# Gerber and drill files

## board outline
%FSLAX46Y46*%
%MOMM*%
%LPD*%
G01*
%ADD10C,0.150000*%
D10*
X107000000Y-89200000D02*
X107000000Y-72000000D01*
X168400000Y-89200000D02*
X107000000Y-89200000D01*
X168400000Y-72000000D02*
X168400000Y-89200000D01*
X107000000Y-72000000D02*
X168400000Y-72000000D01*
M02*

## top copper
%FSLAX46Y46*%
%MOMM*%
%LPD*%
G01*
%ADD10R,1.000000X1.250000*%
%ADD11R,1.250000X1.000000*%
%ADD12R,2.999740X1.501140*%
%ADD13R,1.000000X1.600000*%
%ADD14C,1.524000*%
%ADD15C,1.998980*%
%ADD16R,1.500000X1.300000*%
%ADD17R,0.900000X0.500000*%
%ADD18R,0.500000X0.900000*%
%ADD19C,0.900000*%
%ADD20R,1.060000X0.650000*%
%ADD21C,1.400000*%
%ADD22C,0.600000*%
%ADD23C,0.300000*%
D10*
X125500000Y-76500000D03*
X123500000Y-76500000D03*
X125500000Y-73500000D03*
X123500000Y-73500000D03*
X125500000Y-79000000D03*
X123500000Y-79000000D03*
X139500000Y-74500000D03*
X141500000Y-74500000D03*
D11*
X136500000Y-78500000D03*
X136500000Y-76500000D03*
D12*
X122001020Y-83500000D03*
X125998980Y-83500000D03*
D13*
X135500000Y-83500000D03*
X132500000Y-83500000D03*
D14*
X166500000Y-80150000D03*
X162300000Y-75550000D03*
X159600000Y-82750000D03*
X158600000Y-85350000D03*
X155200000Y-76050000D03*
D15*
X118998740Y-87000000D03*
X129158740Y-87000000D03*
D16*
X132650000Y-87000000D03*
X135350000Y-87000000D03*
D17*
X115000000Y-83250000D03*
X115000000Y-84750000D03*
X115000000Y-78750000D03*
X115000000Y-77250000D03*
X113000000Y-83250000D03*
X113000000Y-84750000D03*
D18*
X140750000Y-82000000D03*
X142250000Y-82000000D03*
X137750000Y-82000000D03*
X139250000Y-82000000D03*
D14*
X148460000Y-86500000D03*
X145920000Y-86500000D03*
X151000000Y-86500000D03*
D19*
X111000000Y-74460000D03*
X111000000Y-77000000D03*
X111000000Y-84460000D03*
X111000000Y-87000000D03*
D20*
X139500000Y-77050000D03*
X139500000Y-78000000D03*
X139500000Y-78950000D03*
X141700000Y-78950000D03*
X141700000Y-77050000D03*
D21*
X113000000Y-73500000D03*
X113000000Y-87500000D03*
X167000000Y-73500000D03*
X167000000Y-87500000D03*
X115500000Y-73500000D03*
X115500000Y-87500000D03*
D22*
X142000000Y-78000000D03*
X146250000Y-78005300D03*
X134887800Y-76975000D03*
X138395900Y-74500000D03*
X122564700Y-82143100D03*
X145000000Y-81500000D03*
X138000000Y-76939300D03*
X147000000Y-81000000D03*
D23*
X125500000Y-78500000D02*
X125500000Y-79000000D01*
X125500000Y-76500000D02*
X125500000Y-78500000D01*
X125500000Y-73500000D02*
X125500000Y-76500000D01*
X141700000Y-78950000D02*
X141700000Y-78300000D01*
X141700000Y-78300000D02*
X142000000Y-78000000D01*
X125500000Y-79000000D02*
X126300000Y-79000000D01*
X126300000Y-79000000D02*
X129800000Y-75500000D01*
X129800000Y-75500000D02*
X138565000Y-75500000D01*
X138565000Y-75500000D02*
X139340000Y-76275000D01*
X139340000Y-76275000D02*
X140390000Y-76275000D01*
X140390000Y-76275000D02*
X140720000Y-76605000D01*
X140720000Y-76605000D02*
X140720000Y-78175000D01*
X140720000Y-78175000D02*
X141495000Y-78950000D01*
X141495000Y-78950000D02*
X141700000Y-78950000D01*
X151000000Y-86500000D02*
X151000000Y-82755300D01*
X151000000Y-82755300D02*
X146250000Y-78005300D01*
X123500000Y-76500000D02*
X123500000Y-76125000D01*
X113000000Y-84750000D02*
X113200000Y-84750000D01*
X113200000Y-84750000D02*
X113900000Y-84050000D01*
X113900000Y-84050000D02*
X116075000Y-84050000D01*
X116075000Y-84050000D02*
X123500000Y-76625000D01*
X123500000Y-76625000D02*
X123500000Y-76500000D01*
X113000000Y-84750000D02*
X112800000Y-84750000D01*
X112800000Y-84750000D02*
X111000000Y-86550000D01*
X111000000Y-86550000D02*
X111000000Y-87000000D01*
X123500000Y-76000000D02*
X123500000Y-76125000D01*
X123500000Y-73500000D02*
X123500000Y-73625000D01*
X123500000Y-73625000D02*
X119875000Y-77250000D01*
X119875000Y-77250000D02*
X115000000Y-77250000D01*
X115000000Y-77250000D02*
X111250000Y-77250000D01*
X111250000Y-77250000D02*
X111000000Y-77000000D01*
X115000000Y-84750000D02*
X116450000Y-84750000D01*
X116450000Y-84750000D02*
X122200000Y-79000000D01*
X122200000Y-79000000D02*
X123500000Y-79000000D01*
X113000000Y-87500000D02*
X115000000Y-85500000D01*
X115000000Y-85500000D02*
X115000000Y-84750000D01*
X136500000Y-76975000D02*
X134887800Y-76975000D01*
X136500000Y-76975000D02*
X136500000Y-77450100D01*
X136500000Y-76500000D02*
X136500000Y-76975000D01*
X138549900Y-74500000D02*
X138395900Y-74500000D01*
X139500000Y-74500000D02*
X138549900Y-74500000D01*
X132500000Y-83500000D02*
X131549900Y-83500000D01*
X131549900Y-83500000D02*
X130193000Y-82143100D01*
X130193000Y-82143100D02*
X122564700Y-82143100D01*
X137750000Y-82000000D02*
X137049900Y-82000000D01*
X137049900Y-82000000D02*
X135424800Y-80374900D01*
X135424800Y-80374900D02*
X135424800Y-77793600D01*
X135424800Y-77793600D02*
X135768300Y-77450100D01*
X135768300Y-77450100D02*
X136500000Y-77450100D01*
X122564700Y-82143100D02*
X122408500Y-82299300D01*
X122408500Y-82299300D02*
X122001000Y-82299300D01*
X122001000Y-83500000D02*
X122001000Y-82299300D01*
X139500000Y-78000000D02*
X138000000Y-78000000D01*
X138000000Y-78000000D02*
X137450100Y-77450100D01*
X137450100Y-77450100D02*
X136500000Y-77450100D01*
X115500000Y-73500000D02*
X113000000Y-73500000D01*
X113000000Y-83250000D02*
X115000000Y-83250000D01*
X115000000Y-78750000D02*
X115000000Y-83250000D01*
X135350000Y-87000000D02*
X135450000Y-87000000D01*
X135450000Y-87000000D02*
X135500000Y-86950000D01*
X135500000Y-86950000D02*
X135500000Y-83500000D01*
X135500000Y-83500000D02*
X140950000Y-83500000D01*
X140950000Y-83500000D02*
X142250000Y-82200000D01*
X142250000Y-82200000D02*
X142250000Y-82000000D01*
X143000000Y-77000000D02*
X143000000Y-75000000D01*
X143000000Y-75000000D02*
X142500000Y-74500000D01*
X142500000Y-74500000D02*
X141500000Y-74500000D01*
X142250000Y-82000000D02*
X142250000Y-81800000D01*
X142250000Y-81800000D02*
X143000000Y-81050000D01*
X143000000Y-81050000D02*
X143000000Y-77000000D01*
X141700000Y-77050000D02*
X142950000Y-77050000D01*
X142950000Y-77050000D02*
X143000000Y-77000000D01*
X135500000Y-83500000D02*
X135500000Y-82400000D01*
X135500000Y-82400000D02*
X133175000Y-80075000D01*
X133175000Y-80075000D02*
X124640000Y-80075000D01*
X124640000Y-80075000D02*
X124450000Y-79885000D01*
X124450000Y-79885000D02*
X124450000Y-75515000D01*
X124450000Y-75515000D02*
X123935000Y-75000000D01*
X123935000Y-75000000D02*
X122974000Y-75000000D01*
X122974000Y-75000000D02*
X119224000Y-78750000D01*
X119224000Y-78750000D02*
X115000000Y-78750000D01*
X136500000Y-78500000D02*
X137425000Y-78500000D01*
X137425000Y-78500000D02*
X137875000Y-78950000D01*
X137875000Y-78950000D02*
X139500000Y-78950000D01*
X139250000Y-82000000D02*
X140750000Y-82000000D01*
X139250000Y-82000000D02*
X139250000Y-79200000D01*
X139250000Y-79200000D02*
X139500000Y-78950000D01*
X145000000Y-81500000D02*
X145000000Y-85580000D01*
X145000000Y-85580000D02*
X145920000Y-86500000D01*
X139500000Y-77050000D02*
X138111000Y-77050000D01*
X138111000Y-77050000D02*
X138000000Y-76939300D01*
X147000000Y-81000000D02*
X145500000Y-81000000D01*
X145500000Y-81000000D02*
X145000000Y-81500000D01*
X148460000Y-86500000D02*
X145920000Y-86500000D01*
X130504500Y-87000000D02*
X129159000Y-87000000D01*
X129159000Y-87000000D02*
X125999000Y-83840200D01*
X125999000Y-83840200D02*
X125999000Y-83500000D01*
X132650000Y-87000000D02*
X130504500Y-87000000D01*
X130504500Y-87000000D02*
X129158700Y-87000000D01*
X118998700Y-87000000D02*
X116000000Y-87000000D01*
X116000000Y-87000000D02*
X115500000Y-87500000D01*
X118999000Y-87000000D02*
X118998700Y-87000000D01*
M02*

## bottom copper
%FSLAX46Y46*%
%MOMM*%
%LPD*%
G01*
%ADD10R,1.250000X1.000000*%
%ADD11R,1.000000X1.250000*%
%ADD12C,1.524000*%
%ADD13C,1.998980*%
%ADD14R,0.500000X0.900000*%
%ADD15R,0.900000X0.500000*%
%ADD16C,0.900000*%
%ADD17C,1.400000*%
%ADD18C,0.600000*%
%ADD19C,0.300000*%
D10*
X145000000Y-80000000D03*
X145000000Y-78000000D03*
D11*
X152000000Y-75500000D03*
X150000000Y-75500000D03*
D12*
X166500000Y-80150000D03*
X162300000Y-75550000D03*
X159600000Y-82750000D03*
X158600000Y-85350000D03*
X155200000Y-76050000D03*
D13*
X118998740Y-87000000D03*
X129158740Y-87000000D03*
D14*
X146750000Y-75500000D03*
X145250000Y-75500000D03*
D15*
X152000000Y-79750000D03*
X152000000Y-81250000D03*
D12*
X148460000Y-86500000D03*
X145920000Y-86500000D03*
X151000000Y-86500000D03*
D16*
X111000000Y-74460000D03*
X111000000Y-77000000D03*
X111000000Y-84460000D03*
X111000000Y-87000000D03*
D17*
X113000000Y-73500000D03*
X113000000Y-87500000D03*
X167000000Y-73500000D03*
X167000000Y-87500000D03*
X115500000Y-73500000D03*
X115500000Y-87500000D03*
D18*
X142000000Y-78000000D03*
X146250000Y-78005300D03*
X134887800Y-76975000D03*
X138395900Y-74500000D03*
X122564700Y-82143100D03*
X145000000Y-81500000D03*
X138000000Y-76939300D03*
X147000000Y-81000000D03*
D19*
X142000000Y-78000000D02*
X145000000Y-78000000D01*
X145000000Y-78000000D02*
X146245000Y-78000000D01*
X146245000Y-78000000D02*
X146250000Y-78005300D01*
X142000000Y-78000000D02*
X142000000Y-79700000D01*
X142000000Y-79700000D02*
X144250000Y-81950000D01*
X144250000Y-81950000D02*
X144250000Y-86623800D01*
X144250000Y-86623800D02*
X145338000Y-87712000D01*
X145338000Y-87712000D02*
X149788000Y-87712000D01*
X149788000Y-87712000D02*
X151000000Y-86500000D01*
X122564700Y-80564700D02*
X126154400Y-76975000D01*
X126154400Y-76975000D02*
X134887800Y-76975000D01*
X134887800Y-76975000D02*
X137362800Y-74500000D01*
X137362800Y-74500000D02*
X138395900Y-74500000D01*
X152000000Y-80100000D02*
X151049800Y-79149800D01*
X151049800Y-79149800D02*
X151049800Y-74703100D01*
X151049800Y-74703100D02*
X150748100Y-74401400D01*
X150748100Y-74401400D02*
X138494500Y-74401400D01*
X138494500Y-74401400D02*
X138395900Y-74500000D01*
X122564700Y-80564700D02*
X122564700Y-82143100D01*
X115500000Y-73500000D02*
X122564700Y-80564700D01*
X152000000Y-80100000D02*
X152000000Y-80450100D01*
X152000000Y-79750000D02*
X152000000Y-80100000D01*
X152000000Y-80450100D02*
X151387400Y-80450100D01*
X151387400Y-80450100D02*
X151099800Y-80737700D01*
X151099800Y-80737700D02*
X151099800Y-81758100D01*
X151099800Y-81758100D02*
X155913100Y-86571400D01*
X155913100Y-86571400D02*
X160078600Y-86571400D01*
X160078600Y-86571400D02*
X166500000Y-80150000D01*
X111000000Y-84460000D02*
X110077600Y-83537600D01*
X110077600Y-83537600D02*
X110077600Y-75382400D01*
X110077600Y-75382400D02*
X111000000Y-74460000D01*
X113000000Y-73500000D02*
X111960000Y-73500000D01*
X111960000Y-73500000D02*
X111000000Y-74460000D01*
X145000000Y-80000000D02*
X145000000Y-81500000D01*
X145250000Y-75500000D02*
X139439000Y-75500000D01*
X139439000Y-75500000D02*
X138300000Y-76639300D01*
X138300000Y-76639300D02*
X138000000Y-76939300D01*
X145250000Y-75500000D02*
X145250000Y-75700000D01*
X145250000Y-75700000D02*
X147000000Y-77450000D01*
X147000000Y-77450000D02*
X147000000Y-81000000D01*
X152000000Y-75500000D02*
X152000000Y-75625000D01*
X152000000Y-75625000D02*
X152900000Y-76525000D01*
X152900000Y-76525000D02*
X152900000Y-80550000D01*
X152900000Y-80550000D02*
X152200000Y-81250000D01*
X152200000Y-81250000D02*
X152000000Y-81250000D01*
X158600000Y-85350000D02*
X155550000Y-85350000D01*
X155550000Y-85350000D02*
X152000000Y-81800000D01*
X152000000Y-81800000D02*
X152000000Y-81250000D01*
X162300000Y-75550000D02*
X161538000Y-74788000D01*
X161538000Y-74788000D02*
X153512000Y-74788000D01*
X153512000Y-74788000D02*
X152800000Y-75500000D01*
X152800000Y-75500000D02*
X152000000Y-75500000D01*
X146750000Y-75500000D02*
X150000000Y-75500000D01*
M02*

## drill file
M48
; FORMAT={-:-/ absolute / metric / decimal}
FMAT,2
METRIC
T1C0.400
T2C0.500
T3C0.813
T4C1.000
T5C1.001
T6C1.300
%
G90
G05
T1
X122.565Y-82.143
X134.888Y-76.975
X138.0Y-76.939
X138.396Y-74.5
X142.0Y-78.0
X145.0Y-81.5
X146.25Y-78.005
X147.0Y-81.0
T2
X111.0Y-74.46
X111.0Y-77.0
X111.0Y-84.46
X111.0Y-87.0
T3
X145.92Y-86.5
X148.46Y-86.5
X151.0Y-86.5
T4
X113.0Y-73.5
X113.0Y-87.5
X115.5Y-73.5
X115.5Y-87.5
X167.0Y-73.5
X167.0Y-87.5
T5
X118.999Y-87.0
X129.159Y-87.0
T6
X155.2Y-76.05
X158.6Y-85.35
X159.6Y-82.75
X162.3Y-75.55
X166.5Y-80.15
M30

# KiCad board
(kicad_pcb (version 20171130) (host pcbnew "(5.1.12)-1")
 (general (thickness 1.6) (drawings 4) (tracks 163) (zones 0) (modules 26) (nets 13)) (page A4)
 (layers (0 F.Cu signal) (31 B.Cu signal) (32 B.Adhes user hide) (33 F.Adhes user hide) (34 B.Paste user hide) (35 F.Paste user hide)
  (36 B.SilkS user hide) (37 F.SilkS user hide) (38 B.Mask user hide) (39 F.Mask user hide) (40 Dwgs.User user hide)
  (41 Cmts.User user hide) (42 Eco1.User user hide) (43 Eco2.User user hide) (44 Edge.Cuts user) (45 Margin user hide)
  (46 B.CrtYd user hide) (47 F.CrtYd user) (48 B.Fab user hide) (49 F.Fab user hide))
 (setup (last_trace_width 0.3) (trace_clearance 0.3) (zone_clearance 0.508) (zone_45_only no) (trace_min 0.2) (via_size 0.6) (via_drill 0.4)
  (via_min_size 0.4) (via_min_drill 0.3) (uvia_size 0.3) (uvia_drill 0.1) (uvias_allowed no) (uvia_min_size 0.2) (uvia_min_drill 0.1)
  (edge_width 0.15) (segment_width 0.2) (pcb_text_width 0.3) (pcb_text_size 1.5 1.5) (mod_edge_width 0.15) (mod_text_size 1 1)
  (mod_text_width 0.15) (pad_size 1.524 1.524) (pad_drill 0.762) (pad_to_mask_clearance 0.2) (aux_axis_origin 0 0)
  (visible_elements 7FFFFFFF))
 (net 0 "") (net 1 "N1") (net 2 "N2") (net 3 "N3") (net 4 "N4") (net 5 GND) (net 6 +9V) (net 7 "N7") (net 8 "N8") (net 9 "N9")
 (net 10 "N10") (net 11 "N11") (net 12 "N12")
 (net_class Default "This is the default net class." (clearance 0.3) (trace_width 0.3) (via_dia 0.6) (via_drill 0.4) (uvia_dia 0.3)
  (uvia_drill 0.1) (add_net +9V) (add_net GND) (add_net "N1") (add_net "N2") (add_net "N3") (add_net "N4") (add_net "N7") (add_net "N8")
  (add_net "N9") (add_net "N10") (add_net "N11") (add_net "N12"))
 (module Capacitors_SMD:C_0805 (layer F.Cu) (at 124.5 76.5 180)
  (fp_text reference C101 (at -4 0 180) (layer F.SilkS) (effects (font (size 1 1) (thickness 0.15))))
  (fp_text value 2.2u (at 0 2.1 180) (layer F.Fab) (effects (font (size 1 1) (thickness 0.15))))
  (pad 1 smd rect (at -1 0 180) (size 1 1.25) (layers F.Cu F.Paste F.Mask) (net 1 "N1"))
  (pad 2 smd rect (at 1 0 180) (size 1 1.25) (layers F.Cu F.Paste F.Mask) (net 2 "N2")))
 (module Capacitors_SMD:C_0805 (layer F.Cu) (at 124.5 73.5 180)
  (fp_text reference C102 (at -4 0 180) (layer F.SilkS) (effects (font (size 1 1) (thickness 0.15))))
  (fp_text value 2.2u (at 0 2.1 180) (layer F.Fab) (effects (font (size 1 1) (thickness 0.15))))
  (pad 1 smd rect (at -1 0 180) (size 1 1.25) (layers F.Cu F.Paste F.Mask) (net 1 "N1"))
  (pad 2 smd rect (at 1 0 180) (size 1 1.25) (layers F.Cu F.Paste F.Mask) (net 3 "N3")))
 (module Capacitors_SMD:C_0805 (layer F.Cu) (at 124.5 79 180)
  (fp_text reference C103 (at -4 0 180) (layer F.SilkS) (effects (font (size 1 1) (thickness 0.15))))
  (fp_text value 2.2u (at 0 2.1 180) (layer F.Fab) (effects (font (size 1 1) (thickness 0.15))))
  (pad 1 smd rect (at -1 0 180) (size 1 1.25) (layers F.Cu F.Paste F.Mask) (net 1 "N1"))
  (pad 2 smd rect (at 1 0 180) (size 1 1.25) (layers F.Cu F.Paste F.Mask) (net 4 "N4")))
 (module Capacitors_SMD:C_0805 (layer F.Cu) (at 140.5 74.5)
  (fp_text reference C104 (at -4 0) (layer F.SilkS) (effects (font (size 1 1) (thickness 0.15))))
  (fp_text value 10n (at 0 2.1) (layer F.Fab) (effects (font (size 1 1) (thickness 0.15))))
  (pad 1 smd rect (at -1 0) (size 1 1.25) (layers F.Cu F.Paste F.Mask) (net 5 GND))
  (pad 2 smd rect (at 1 0) (size 1 1.25) (layers F.Cu F.Paste F.Mask) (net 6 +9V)))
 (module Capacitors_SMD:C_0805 (layer F.Cu) (at 136.5 77.5 90)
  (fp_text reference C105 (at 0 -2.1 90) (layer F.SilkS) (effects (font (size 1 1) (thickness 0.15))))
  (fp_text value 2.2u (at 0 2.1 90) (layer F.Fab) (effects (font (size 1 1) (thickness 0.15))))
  (pad 1 smd rect (at -1 0 90) (size 1 1.25) (layers F.Cu F.Paste F.Mask) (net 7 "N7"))
  (pad 2 smd rect (at 1 0 90) (size 1 1.25) (layers F.Cu F.Paste F.Mask) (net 5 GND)))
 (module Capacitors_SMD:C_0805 (layer B.Cu) (at 145 79 90)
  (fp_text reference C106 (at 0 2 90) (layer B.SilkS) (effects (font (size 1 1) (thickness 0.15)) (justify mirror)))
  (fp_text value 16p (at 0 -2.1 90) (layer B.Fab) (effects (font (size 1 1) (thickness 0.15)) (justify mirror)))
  (pad 1 smd rect (at -1 0 90) (size 1 1.25) (layers B.Cu B.Paste B.Mask) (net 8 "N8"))
  (pad 2 smd rect (at 1 0 90) (size 1 1.25) (layers B.Cu B.Paste B.Mask) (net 1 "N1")))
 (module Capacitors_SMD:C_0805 (layer B.Cu) (at 151 75.5 180)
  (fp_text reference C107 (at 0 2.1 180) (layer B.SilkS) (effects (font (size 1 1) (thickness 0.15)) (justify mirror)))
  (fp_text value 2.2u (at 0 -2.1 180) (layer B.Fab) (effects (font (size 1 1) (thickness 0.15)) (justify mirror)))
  (pad 1 smd rect (at -1 0 180) (size 1 1.25) (layers B.Cu B.Paste B.Mask) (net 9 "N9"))
  (pad 2 smd rect (at 1 0 180) (size 1 1.25) (layers B.Cu B.Paste B.Mask) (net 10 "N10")))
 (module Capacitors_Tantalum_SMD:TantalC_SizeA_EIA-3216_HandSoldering (layer F.Cu) (at 124 83.5 180)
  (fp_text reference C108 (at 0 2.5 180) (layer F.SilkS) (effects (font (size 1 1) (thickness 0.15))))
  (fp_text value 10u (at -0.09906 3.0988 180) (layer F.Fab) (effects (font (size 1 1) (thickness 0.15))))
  (pad 2 smd rect (at 1.99898 0 180) (size 2.99974 1.50114) (layers F.Cu F.Paste F.Mask) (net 5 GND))
  (pad 1 smd rect (at -1.99898 0 180) (size 2.99974 1.50114) (layers F.Cu F.Paste F.Mask) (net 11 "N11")))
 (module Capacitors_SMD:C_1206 (layer F.Cu) (at 134 83.5 180)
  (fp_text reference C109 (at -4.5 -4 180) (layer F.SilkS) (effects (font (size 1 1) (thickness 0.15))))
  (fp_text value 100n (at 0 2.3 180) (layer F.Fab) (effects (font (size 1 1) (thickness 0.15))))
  (pad 1 smd rect (at -1.5 0 180) (size 1 1.6) (layers F.Cu F.Paste F.Mask) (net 6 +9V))
  (pad 2 smd rect (at 1.5 0 180) (size 1 1.6) (layers F.Cu F.Paste F.Mask) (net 5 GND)))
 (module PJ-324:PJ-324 (layer F.Cu) (at 168.2 86.15 180)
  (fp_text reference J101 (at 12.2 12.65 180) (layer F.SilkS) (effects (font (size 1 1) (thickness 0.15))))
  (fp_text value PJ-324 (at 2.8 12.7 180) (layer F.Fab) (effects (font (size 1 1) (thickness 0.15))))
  (pad 1 thru_hole circle (at 1.7 6 180) (size 1.524 1.524) (drill 1.3) (layers *.Cu *.Mask) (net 5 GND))
  (pad 5 thru_hole circle (at 5.9 10.6 180) (size 1.524 1.524) (drill 1.3) (layers *.Cu *.Mask) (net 9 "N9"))
  (pad 3 thru_hole circle (at 8.6 3.4 180) (size 1.524 1.524) (drill 1.3) (layers *.Cu *.Mask))
  (pad 2 thru_hole circle (at 9.6 0.8 180) (size 1.524 1.524) (drill 1.3) (layers *.Cu *.Mask) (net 9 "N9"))
  (pad 4 thru_hole circle (at 13 10.1 180) (size 1.524 1.524) (drill 1.3) (layers *.Cu *.Mask)))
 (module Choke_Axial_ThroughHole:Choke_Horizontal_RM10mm (layer F.Cu) (at 124 87)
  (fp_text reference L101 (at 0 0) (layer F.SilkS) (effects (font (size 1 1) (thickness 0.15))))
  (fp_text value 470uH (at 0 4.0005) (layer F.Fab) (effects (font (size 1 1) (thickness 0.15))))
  (pad 1 thru_hole circle (at -5.00126 0) (size 1.99898 1.99898) (drill 1.00076) (layers *.Cu *.Mask F.SilkS) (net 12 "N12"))
  (pad 2 thru_hole circle (at 5.15874 0) (size 1.99898 1.99898) (drill 1.00076) (layers *.Cu *.Mask F.SilkS) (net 11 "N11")))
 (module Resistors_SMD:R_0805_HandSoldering (layer F.Cu) (at 134 87)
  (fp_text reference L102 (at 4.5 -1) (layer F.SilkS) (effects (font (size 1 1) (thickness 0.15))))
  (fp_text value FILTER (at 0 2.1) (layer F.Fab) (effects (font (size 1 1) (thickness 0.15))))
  (pad 1 smd rect (at -1.35 0) (size 1.5 1.3) (layers F.Cu F.Paste F.Mask) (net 11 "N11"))
  (pad 2 smd rect (at 1.35 0) (size 1.5 1.3) (layers F.Cu F.Paste F.Mask) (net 6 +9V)))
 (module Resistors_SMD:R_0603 (layer F.Cu) (at 115 84 270)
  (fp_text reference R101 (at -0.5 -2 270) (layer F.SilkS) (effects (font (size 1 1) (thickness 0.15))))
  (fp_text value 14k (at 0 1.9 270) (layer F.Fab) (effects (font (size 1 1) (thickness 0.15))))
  (pad 1 smd rect (at -0.75 0 270) (size 0.5 0.9) (layers F.Cu F.Paste F.Mask) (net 6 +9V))
  (pad 2 smd rect (at 0.75 0 270) (size 0.5 0.9) (layers F.Cu F.Paste F.Mask) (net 4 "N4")))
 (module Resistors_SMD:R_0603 (layer F.Cu) (at 115 78 90)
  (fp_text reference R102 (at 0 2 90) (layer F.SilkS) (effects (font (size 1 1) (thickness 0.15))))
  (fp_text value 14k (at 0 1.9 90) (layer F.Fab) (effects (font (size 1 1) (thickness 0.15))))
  (pad 1 smd rect (at -0.75 0 90) (size 0.5 0.9) (layers F.Cu F.Paste F.Mask) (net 6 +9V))
  (pad 2 smd rect (at 0.75 0 90) (size 0.5 0.9) (layers F.Cu F.Paste F.Mask) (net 3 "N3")))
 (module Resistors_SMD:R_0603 (layer F.Cu) (at 113 84 270)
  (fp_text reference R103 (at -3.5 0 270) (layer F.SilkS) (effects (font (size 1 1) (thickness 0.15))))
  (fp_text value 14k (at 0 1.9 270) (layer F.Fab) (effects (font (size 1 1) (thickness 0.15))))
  (pad 1 smd rect (at -0.75 0 270) (size 0.5 0.9) (layers F.Cu F.Paste F.Mask) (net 6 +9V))
  (pad 2 smd rect (at 0.75 0 270) (size 0.5 0.9) (layers F.Cu F.Paste F.Mask) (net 2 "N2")))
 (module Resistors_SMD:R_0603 (layer F.Cu) (at 141.5 82)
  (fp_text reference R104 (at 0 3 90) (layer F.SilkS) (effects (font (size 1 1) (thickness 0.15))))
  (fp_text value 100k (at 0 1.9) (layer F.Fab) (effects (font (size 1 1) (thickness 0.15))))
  (pad 1 smd rect (at -0.75 0) (size 0.5 0.9) (layers F.Cu F.Paste F.Mask) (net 7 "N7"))
  (pad 2 smd rect (at 0.75 0) (size 0.5 0.9) (layers F.Cu F.Paste F.Mask) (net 6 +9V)))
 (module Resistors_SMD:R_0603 (layer F.Cu) (at 138.5 82)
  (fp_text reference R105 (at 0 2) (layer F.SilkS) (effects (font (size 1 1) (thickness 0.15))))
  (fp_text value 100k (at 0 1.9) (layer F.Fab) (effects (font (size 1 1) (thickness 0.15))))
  (pad 1 smd rect (at -0.75 0) (size 0.5 0.9) (layers F.Cu F.Paste F.Mask) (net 5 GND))
  (pad 2 smd rect (at 0.75 0) (size 0.5 0.9) (layers F.Cu F.Paste F.Mask) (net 7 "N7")))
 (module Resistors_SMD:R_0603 (layer B.Cu) (at 146 75.5 180)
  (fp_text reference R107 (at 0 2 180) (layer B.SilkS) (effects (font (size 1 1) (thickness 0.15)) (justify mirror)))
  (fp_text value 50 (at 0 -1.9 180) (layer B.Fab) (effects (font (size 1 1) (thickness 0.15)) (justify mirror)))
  (pad 1 smd rect (at -0.75 0 180) (size 0.5 0.9) (layers B.Cu B.Paste B.Mask) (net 10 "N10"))
  (pad 2 smd rect (at 0.75 0 180) (size 0.5 0.9) (layers B.Cu B.Paste B.Mask) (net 8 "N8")))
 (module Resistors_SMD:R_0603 (layer B.Cu) (at 152 80.5 270)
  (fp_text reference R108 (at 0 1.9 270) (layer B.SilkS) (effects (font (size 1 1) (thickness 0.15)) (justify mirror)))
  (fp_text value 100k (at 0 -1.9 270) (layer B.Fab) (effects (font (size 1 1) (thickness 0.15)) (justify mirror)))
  (pad 1 smd rect (at -0.75 0 270) (size 0.5 0.9) (layers B.Cu B.Paste B.Mask) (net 5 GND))
  (pad 2 smd rect (at 0.75 0 270) (size 0.5 0.9) (layers B.Cu B.Paste B.Mask) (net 9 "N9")))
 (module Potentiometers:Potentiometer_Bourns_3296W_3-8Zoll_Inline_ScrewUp (layer F.Cu) (at 151 86.5 90)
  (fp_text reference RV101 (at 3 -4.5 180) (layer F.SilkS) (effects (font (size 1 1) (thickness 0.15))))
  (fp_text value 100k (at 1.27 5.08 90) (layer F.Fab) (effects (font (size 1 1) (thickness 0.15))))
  (pad 2 thru_hole circle (at 0 -2.54 90) (size 1.524 1.524) (drill 0.8128) (layers *.Cu *.Mask F.SilkS) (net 8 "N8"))
  (pad 3 thru_hole circle (at 0 -5.08 90) (size 1.524 1.524) (drill 0.8128) (layers *.Cu *.Mask F.SilkS) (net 8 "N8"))
  (pad 1 thru_hole circle (at 0 0 90) (size 1.524 1.524) (drill 0.8128) (layers *.Cu *.Mask F.SilkS) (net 1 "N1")))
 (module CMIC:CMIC (layer F.Cu) (at 111 80.48 90)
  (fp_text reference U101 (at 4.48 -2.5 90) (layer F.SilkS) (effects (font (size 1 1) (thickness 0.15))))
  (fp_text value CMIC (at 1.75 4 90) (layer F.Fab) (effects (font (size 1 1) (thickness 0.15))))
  (pad 2 thru_hole circle (at 6.02 0 90) (size 0.9 0.9) (drill 0.5) (layers *.Cu *.Mask) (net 5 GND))
  (pad 1 thru_hole circle (at 3.48 0 90) (size 0.9 0.9) (drill 0.5) (layers *.Cu *.Mask) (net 3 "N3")))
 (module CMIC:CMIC (layer F.Cu) (at 111 90.48 90)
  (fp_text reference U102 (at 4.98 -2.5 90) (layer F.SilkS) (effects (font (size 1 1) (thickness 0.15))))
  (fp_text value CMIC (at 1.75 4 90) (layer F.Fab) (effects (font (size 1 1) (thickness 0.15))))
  (pad 2 thru_hole circle (at 6.02 0 90) (size 0.9 0.9) (drill 0.5) (layers *.Cu *.Mask) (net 5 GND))
  (pad 1 thru_hole circle (at 3.48 0 90) (size 0.9 0.9) (drill 0.5) (layers *.Cu *.Mask) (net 2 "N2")))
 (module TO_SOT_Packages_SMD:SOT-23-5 (layer F.Cu) (at 140.6 78)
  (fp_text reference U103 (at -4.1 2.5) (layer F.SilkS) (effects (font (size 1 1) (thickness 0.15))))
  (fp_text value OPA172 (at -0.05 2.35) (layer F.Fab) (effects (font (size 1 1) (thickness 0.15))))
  (pad 1 smd rect (at -1.1 -0.95) (size 1.06 0.65) (layers F.Cu F.Paste F.Mask) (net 8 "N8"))
  (pad 2 smd rect (at -1.1 0) (size 1.06 0.65) (layers F.Cu F.Paste F.Mask) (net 5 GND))
  (pad 3 smd rect (at -1.1 0.95) (size 1.06 0.65) (layers F.Cu F.Paste F.Mask) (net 7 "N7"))
  (pad 4 smd rect (at 1.1 0.95) (size 1.06 0.65) (layers F.Cu F.Paste F.Mask) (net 1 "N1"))
  (pad 5 smd rect (at 1.1 -0.95) (size 1.06 0.65) (layers F.Cu F.Paste F.Mask) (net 6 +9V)))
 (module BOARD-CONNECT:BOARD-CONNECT (layer F.Cu) (at 113 73)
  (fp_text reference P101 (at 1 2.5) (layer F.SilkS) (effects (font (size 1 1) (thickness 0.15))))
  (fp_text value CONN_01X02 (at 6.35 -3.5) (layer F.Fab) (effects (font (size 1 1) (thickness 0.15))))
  (pad 1 thru_hole circle (at 0 0.5) (size 1.4 1.4) (drill 1) (layers *.Cu *.Mask) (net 5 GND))
  (pad 2 thru_hole circle (at 0 14.5) (size 1.4 1.4) (drill 1) (layers *.Cu *.Mask) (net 4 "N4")))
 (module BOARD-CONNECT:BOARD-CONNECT (layer F.Cu) (at 167 73)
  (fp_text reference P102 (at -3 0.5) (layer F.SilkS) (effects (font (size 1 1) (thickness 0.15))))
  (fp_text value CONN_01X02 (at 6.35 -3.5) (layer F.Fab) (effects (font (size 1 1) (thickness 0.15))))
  (pad 1 thru_hole circle (at 0 0.5) (size 1.4 1.4) (drill 1) (layers *.Cu *.Mask))
  (pad 2 thru_hole circle (at 0 14.5) (size 1.4 1.4) (drill 1) (layers *.Cu *.Mask)))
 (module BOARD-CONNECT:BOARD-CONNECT (layer F.Cu) (at 115.5 73)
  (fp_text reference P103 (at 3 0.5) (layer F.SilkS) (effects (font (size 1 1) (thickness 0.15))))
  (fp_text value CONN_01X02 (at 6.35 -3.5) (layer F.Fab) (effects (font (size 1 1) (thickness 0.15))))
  (pad 1 thru_hole circle (at 0 0.5) (size 1.4 1.4) (drill 1) (layers *.Cu *.Mask) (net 5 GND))
  (pad 2 thru_hole circle (at 0 14.5) (size 1.4 1.4) (drill 1) (layers *.Cu *.Mask) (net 12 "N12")))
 (gr_line (start 107 89.2) (end 107 72) (layer Edge.Cuts) (width 0.15))
 (gr_line (start 168.4 89.2) (end 107 89.2) (layer Edge.Cuts) (width 0.15))
 (gr_line (start 168.4 72) (end 168.4 89.2) (layer Edge.Cuts) (width 0.15))
 (gr_line (start 107 72) (end 168.4 72) (layer Edge.Cuts) (width 0.15))
 (segment (start 125.5 78.5) (end 125.5 79) (width 0.3) (layer F.Cu) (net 1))
 (segment (start 125.5 76.5) (end 125.5 78.5) (width 0.3) (layer F.Cu) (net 1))
 (segment (start 125.5 73.5) (end 125.5 76.5) (width 0.3) (layer F.Cu) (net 1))
 (segment (start 141.7 78.95) (end 141.7 78.3) (width 0.3) (layer F.Cu) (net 1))
 (segment (start 141.7 78.3) (end 142 78) (width 0.3) (layer F.Cu) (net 1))
 (segment (start 142 78) (end 145 78) (width 0.3) (layer B.Cu) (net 1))
 (segment (start 125.5 79) (end 126.3 79) (width 0.3) (layer F.Cu) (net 1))
 (segment (start 126.3 79) (end 129.8 75.5) (width 0.3) (layer F.Cu) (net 1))
 (segment (start 129.8 75.5) (end 138.565 75.5) (width 0.3) (layer F.Cu) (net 1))
 (segment (start 138.565 75.5) (end 139.34 76.275) (width 0.3) (layer F.Cu) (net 1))
 (segment (start 139.34 76.275) (end 140.39 76.275) (width 0.3) (layer F.Cu) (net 1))
 (segment (start 140.39 76.275) (end 140.72 76.605) (width 0.3) (layer F.Cu) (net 1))
 (segment (start 140.72 76.605) (end 140.72 78.175) (width 0.3) (layer F.Cu) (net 1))
 (segment (start 140.72 78.175) (end 141.495 78.95) (width 0.3) (layer F.Cu) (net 1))
 (segment (start 141.495 78.95) (end 141.7 78.95) (width 0.3) (layer F.Cu) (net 1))
 (segment (start 145 78) (end 146.245 78) (width 0.3) (layer B.Cu) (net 1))
 (segment (start 146.245 78) (end 146.25 78.0053) (width 0.3) (layer B.Cu) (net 1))
 (segment (start 151 86.5) (end 151 82.7553) (width 0.3) (layer F.Cu) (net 1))
 (segment (start 151 82.7553) (end 146.25 78.0053) (width 0.3) (layer F.Cu) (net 1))
 (segment (start 142 78) (end 142 79.7) (width 0.3) (layer B.Cu) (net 1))
 (segment (start 142 79.7) (end 144.25 81.95) (width 0.3) (layer B.Cu) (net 1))
 (segment (start 144.25 81.95) (end 144.25 86.6238) (width 0.3) (layer B.Cu) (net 1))
 (segment (start 144.25 86.6238) (end 145.338 87.712) (width 0.3) (layer B.Cu) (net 1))
 (segment (start 145.338 87.712) (end 149.788 87.712) (width 0.3) (layer B.Cu) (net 1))
 (segment (start 149.788 87.712) (end 151 86.5) (width 0.3) (layer B.Cu) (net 1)) (via (at 142 78) (size 0.6) (layers F.Cu B.Cu) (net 1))
 (via (at 146.25 78.0053) (size 0.6) (layers F.Cu B.Cu) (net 1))
 (segment (start 123.5 76.5) (end 123.5 76.125) (width 0.3) (layer F.Cu) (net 2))
 (segment (start 113 84.75) (end 113.2 84.75) (width 0.3) (layer F.Cu) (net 2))
 (segment (start 113.2 84.75) (end 113.9 84.05) (width 0.3) (layer F.Cu) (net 2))
 (segment (start 113.9 84.05) (end 116.075 84.05) (width 0.3) (layer F.Cu) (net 2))
 (segment (start 116.075 84.05) (end 123.5 76.625) (width 0.3) (layer F.Cu) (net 2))
 (segment (start 123.5 76.625) (end 123.5 76.5) (width 0.3) (layer F.Cu) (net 2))
 (segment (start 113 84.75) (end 112.8 84.75) (width 0.3) (layer F.Cu) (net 2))
 (segment (start 112.8 84.75) (end 111 86.55) (width 0.3) (layer F.Cu) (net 2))
 (segment (start 111 86.55) (end 111 87) (width 0.3) (layer F.Cu) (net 2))
 (segment (start 123.5 76) (end 123.5 76.125) (width 0.3) (layer F.Cu) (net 2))
 (segment (start 123.5 73.5) (end 123.5 73.625) (width 0.3) (layer F.Cu) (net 3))
 (segment (start 123.5 73.625) (end 119.875 77.25) (width 0.3) (layer F.Cu) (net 3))
 (segment (start 119.875 77.25) (end 115 77.25) (width 0.3) (layer F.Cu) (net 3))
 (segment (start 115 77.25) (end 111.25 77.25) (width 0.3) (layer F.Cu) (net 3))
 (segment (start 111.25 77.25) (end 111 77) (width 0.3) (layer F.Cu) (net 3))
 (segment (start 115 84.75) (end 116.45 84.75) (width 0.3) (layer F.Cu) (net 4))
 (segment (start 116.45 84.75) (end 122.2 79) (width 0.3) (layer F.Cu) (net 4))
 (segment (start 122.2 79) (end 123.5 79) (width 0.3) (layer F.Cu) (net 4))
 (segment (start 113 87.5) (end 115 85.5) (width 0.3) (layer F.Cu) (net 4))
 (segment (start 115 85.5) (end 115 84.75) (width 0.3) (layer F.Cu) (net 4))
 (segment (start 122.5647 80.5647) (end 126.1544 76.975) (width 0.3) (layer B.Cu) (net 5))
 (segment (start 126.1544 76.975) (end 134.8878 76.975) (width 0.3) (layer B.Cu) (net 5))
 (segment (start 134.8878 76.975) (end 137.3628 74.5) (width 0.3) (layer B.Cu) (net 5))
 (segment (start 137.3628 74.5) (end 138.3959 74.5) (width 0.3) (layer B.Cu) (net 5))
 (segment (start 136.5 76.975) (end 134.8878 76.975) (width 0.3) (layer F.Cu) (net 5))
 (segment (start 136.5 76.975) (end 136.5 77.4501) (width 0.3) (layer F.Cu) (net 5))
 (segment (start 136.5 76.5) (end 136.5 76.975) (width 0.3) (layer F.Cu) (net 5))
 (segment (start 138.5499 74.5) (end 138.3959 74.5) (width 0.3) (layer F.Cu) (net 5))
 (segment (start 152 80.1) (end 151.0498 79.1498) (width 0.3) (layer B.Cu) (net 5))
 (segment (start 151.0498 79.1498) (end 151.0498 74.7031) (width 0.3) (layer B.Cu) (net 5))
 (segment (start 151.0498 74.7031) (end 150.7481 74.4014) (width 0.3) (layer B.Cu) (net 5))
 (segment (start 150.7481 74.4014) (end 138.4945 74.4014) (width 0.3) (layer B.Cu) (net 5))
 (segment (start 138.4945 74.4014) (end 138.3959 74.5) (width 0.3) (layer B.Cu) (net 5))
 (segment (start 139.5 74.5) (end 138.5499 74.5) (width 0.3) (layer F.Cu) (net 5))
 (segment (start 132.5 83.5) (end 131.5499 83.5) (width 0.3) (layer F.Cu) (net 5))
 (segment (start 131.5499 83.5) (end 130.193 82.1431) (width 0.3) (layer F.Cu) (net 5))
 (segment (start 130.193 82.1431) (end 122.5647 82.1431) (width 0.3) (layer F.Cu) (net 5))
 (segment (start 122.5647 80.5647) (end 122.5647 82.1431) (width 0.3) (layer B.Cu) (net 5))
 (segment (start 115.5 73.5) (end 122.5647 80.5647) (width 0.3) (layer B.Cu) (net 5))
 (segment (start 152 80.1) (end 152 80.4501) (width 0.3) (layer B.Cu) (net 5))
 (segment (start 152 79.75) (end 152 80.1) (width 0.3) (layer B.Cu) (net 5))
 (segment (start 137.75 82) (end 137.0499 82) (width 0.3) (layer F.Cu) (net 5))
 (segment (start 137.0499 82) (end 135.4248 80.3749) (width 0.3) (layer F.Cu) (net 5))
 (segment (start 135.4248 80.3749) (end 135.4248 77.7936) (width 0.3) (layer F.Cu) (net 5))
 (segment (start 135.4248 77.7936) (end 135.7683 77.4501) (width 0.3) (layer F.Cu) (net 5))
 (segment (start 135.7683 77.4501) (end 136.5 77.4501) (width 0.3) (layer F.Cu) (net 5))
 (segment (start 152 80.4501) (end 151.3874 80.4501) (width 0.3) (layer B.Cu) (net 5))
 (segment (start 151.3874 80.4501) (end 151.0998 80.7377) (width 0.3) (layer B.Cu) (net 5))
 (segment (start 151.0998 80.7377) (end 151.0998 81.7581) (width 0.3) (layer B.Cu) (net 5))
 (segment (start 151.0998 81.7581) (end 155.9131 86.5714) (width 0.3) (layer B.Cu) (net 5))
 (segment (start 155.9131 86.5714) (end 160.0786 86.5714) (width 0.3) (layer B.Cu) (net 5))
 (segment (start 160.0786 86.5714) (end 166.5 80.15) (width 0.3) (layer B.Cu) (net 5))
 (segment (start 122.5647 82.1431) (end 122.4085 82.2993) (width 0.3) (layer F.Cu) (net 5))
 (segment (start 122.4085 82.2993) (end 122.001 82.2993) (width 0.3) (layer F.Cu) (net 5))
 (segment (start 122.001 83.5) (end 122.001 82.2993) (width 0.3) (layer F.Cu) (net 5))
 (segment (start 111 84.46) (end 110.0776 83.5376) (width 0.3) (layer B.Cu) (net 5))
 (segment (start 110.0776 83.5376) (end 110.0776 75.3824) (width 0.3) (layer B.Cu) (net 5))
 (segment (start 110.0776 75.3824) (end 111 74.46) (width 0.3) (layer B.Cu) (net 5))
 (segment (start 139.5 78) (end 138 78) (width 0.3) (layer F.Cu) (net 5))
 (segment (start 138 78) (end 137.4501 77.4501) (width 0.3) (layer F.Cu) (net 5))
 (segment (start 137.4501 77.4501) (end 136.5 77.4501) (width 0.3) (layer F.Cu) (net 5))
 (segment (start 113 73.5) (end 111.96 73.5) (width 0.3) (layer B.Cu) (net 5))
 (segment (start 111.96 73.5) (end 111 74.46) (width 0.3) (layer B.Cu) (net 5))
 (segment (start 115.5 73.5) (end 113 73.5) (width 0.3) (layer F.Cu) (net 5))
 (via (at 134.8878 76.975) (size 0.6) (layers F.Cu B.Cu) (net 5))
 (via (at 138.3959 74.5) (size 0.6) (layers F.Cu B.Cu) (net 5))
 (via (at 122.5647 82.1431) (size 0.6) (layers F.Cu B.Cu) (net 5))
 (segment (start 113 83.25) (end 115 83.25) (width 0.3) (layer F.Cu) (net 6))
 (segment (start 115 78.75) (end 115 83.25) (width 0.3) (layer F.Cu) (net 6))
 (segment (start 135.35 87) (end 135.45 87) (width 0.3) (layer F.Cu) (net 6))
 (segment (start 135.45 87) (end 135.5 86.95) (width 0.3) (layer F.Cu) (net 6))
 (segment (start 135.5 86.95) (end 135.5 83.5) (width 0.3) (layer F.Cu) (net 6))
 (segment (start 135.5 83.5) (end 140.95 83.5) (width 0.3) (layer F.Cu) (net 6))
 (segment (start 140.95 83.5) (end 142.25 82.2) (width 0.3) (layer F.Cu) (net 6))
 (segment (start 142.25 82.2) (end 142.25 82) (width 0.3) (layer F.Cu) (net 6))
 (segment (start 143 77) (end 143 75) (width 0.3) (layer F.Cu) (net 6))
 (segment (start 143 75) (end 142.5 74.5) (width 0.3) (layer F.Cu) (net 6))
 (segment (start 142.5 74.5) (end 141.5 74.5) (width 0.3) (layer F.Cu) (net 6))
 (segment (start 142.25 82) (end 142.25 81.8) (width 0.3) (layer F.Cu) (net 6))
 (segment (start 142.25 81.8) (end 143 81.05) (width 0.3) (layer F.Cu) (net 6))
 (segment (start 143 81.05) (end 143 77) (width 0.3) (layer F.Cu) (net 6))
 (segment (start 141.7 77.05) (end 142.95 77.05) (width 0.3) (layer F.Cu) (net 6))
 (segment (start 142.95 77.05) (end 143 77) (width 0.3) (layer F.Cu) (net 6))
 (segment (start 135.5 83.5) (end 135.5 82.4) (width 0.3) (layer F.Cu) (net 6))
 (segment (start 135.5 82.4) (end 133.175 80.075) (width 0.3) (layer F.Cu) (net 6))
 (segment (start 133.175 80.075) (end 124.64 80.075) (width 0.3) (layer F.Cu) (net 6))
 (segment (start 124.64 80.075) (end 124.45 79.885) (width 0.3) (layer F.Cu) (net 6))
 (segment (start 124.45 79.885) (end 124.45 75.515) (width 0.3) (layer F.Cu) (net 6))
 (segment (start 124.45 75.515) (end 123.935 75) (width 0.3) (layer F.Cu) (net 6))
 (segment (start 123.935 75) (end 122.974 75) (width 0.3) (layer F.Cu) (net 6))
 (segment (start 122.974 75) (end 119.224 78.75) (width 0.3) (layer F.Cu) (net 6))
 (segment (start 119.224 78.75) (end 115 78.75) (width 0.3) (layer F.Cu) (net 6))
 (segment (start 136.5 78.5) (end 137.425 78.5) (width 0.3) (layer F.Cu) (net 7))
 (segment (start 137.425 78.5) (end 137.875 78.95) (width 0.3) (layer F.Cu) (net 7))
 (segment (start 137.875 78.95) (end 139.5 78.95) (width 0.3) (layer F.Cu) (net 7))
 (segment (start 139.25 82) (end 140.75 82) (width 0.3) (layer F.Cu) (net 7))
 (segment (start 139.25 82) (end 139.25 79.2) (width 0.3) (layer F.Cu) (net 7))
 (segment (start 139.25 79.2) (end 139.5 78.95) (width 0.3) (layer F.Cu) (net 7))
 (segment (start 145 80) (end 145 81.5) (width 0.3) (layer B.Cu) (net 8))
 (segment (start 145 81.5) (end 145 85.58) (width 0.3) (layer F.Cu) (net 8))
 (segment (start 145 85.58) (end 145.92 86.5) (width 0.3) (layer F.Cu) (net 8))
 (segment (start 139.5 77.05) (end 138.111 77.05) (width 0.3) (layer F.Cu) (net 8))
 (segment (start 138.111 77.05) (end 138 76.9393) (width 0.3) (layer F.Cu) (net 8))
 (segment (start 145.25 75.5) (end 139.439 75.5) (width 0.3) (layer B.Cu) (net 8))
 (segment (start 139.439 75.5) (end 138.3 76.6393) (width 0.3) (layer B.Cu) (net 8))
 (segment (start 138.3 76.6393) (end 138 76.9393) (width 0.3) (layer B.Cu) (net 8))
 (segment (start 145.25 75.5) (end 145.25 75.7) (width 0.3) (layer B.Cu) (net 8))
 (segment (start 145.25 75.7) (end 147 77.45) (width 0.3) (layer B.Cu) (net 8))
 (segment (start 147 77.45) (end 147 81) (width 0.3) (layer B.Cu) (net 8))
 (segment (start 147 81) (end 145.5 81) (width 0.3) (layer F.Cu) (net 8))
 (segment (start 145.5 81) (end 145 81.5) (width 0.3) (layer F.Cu) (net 8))
 (segment (start 148.46 86.5) (end 145.92 86.5) (width 0.3) (layer F.Cu) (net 8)) (via (at 145 81.5) (size 0.6) (layers F.Cu B.Cu) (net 8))
 (via (at 138 76.9393) (size 0.6) (layers F.Cu B.Cu) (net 8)) (via (at 147 81) (size 0.6) (layers F.Cu B.Cu) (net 8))
 (segment (start 152 75.5) (end 152 75.625) (width 0.3) (layer B.Cu) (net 9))
 (segment (start 152 75.625) (end 152.9 76.525) (width 0.3) (layer B.Cu) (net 9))
 (segment (start 152.9 76.525) (end 152.9 80.55) (width 0.3) (layer B.Cu) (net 9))
 (segment (start 152.9 80.55) (end 152.2 81.25) (width 0.3) (layer B.Cu) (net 9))
 (segment (start 152.2 81.25) (end 152 81.25) (width 0.3) (layer B.Cu) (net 9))
 (segment (start 158.6 85.35) (end 155.55 85.35) (width 0.3) (layer B.Cu) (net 9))
 (segment (start 155.55 85.35) (end 152 81.8) (width 0.3) (layer B.Cu) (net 9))
 (segment (start 152 81.8) (end 152 81.25) (width 0.3) (layer B.Cu) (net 9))
 (segment (start 162.3 75.55) (end 161.538 74.788) (width 0.3) (layer B.Cu) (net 9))
 (segment (start 161.538 74.788) (end 153.512 74.788) (width 0.3) (layer B.Cu) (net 9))
 (segment (start 153.512 74.788) (end 152.8 75.5) (width 0.3) (layer B.Cu) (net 9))
 (segment (start 152.8 75.5) (end 152 75.5) (width 0.3) (layer B.Cu) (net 9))
 (segment (start 146.75 75.5) (end 150 75.5) (width 0.3) (layer B.Cu) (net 10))
 (segment (start 130.5045 87) (end 129.159 87) (width 0.3) (layer F.Cu) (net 11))
 (segment (start 129.159 87) (end 125.999 83.8402) (width 0.3) (layer F.Cu) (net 11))
 (segment (start 125.999 83.8402) (end 125.999 83.5) (width 0.3) (layer F.Cu) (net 11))
 (segment (start 132.65 87) (end 130.5045 87) (width 0.3) (layer F.Cu) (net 11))
 (segment (start 130.5045 87) (end 129.1587 87) (width 0.3) (layer F.Cu) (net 11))
 (segment (start 118.9987 87) (end 116 87) (width 0.3) (layer F.Cu) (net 12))
 (segment (start 116 87) (end 115.5 87.5) (width 0.3) (layer F.Cu) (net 12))
 (segment (start 118.999 87) (end 118.9987 87) (width 0.3) (layer F.Cu) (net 12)))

